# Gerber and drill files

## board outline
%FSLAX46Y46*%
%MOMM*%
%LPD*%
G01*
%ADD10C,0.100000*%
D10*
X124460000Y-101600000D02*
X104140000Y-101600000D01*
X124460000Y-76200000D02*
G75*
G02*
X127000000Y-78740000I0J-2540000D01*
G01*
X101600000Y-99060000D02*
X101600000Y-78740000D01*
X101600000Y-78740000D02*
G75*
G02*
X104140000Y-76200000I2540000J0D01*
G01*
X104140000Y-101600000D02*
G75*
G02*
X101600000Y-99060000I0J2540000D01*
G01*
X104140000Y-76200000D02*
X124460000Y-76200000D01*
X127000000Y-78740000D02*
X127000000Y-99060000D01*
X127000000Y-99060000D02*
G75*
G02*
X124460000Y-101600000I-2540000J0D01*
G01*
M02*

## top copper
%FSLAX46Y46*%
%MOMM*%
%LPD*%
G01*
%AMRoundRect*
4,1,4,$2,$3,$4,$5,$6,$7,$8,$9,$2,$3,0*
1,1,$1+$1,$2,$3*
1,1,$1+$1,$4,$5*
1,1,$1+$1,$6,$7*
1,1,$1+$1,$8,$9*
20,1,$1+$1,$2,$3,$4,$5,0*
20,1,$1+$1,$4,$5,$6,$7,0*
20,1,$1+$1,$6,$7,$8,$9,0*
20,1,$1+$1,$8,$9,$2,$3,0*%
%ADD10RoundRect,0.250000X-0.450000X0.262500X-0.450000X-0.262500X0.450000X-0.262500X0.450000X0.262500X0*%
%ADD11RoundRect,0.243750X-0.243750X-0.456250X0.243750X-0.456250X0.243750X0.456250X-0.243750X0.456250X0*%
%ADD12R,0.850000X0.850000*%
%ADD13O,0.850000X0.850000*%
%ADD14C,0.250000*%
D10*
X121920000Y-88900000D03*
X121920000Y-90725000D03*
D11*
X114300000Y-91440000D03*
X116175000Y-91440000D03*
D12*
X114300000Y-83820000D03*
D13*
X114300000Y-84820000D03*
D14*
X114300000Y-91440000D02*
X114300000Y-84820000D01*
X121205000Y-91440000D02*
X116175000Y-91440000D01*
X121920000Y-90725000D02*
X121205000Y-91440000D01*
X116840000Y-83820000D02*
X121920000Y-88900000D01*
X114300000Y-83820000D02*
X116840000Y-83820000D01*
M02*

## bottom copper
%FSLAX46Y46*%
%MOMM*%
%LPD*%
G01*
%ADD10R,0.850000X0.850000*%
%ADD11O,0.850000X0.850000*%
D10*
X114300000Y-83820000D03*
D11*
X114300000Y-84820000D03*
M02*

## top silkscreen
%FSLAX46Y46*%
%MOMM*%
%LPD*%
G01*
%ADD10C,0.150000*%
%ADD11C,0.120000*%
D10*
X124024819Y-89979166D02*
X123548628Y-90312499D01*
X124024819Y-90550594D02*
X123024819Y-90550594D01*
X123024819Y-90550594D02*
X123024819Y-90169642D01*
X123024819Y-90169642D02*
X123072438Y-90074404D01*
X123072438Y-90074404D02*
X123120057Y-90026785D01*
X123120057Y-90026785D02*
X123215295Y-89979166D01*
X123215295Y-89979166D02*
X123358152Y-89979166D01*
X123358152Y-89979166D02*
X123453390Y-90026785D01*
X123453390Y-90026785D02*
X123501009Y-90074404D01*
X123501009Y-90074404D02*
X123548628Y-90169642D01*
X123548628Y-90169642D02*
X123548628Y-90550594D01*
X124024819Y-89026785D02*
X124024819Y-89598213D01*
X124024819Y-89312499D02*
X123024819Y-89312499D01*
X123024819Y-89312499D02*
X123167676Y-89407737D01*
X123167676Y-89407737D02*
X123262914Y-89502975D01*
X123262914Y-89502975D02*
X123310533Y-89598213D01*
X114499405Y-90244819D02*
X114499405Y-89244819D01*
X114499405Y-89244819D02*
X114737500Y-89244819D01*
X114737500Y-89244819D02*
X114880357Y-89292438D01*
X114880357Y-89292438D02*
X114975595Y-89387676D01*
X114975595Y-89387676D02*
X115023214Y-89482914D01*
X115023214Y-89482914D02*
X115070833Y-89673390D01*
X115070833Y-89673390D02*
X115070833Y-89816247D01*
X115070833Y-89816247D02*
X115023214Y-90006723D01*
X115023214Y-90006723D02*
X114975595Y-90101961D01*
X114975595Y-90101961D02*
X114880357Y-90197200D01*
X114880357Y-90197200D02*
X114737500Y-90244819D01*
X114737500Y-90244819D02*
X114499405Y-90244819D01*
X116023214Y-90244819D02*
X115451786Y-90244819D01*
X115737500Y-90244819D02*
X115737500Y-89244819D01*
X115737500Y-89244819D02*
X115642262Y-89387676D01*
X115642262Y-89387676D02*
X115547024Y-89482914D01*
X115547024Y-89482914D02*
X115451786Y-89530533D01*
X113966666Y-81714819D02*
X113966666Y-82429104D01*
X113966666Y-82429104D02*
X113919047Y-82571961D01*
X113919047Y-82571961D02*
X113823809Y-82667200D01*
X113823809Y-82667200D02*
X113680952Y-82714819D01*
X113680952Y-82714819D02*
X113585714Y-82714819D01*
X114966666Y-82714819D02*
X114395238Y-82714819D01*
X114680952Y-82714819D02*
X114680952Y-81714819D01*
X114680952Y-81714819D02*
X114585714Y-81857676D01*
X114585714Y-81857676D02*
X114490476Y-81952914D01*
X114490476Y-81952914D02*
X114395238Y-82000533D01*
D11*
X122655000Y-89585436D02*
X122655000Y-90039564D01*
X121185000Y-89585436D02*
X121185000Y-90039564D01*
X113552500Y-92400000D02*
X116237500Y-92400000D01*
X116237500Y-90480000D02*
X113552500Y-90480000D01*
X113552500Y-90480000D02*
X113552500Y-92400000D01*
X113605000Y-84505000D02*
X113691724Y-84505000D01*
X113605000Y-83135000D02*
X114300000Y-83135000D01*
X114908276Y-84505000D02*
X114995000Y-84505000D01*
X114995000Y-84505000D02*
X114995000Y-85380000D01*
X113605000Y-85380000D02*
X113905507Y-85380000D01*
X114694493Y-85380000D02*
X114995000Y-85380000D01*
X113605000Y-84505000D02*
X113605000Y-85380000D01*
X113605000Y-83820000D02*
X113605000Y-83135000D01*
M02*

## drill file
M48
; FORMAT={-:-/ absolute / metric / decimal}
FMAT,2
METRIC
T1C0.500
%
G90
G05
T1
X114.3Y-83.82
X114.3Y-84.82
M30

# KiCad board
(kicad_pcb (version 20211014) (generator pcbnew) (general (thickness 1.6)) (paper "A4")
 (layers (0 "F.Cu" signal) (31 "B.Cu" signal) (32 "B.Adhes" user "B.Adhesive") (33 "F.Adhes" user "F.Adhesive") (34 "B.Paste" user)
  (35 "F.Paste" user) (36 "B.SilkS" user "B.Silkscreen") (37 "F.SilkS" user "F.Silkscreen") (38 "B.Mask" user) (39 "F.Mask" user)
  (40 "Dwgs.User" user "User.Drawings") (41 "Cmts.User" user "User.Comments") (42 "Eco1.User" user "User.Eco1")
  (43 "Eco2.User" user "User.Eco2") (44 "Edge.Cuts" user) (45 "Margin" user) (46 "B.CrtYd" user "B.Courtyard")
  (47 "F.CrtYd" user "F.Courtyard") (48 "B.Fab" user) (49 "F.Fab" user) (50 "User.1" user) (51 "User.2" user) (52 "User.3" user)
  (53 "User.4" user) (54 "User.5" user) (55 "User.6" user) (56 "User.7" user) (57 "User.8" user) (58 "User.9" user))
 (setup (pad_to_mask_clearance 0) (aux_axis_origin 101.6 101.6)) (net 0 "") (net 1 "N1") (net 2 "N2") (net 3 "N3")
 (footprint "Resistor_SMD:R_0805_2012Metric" (layer "F.Cu") (at 121.92 89.8125 -90)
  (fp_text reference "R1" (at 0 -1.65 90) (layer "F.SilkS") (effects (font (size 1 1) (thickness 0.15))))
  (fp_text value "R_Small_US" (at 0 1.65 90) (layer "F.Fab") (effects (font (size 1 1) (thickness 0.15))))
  (fp_line (start -0.227064 -0.735) (end 0.227064 -0.735) (layer "F.SilkS") (width 0.12))
  (fp_line (start -0.227064 0.735) (end 0.227064 0.735) (layer "F.SilkS") (width 0.12))
  (pad "1" smd roundrect (at -0.9125 0 270) (size 1.025 1.4) (layers "F.Cu" "F.Paste" "F.Mask") (roundrect_rratio 0.243902) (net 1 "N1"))
  (pad "2" smd roundrect (at 0.9125 0 270) (size 1.025 1.4) (layers "F.Cu" "F.Paste" "F.Mask") (roundrect_rratio 0.243902) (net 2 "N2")))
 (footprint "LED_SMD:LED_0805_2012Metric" (layer "F.Cu") (at 115.2375 91.44)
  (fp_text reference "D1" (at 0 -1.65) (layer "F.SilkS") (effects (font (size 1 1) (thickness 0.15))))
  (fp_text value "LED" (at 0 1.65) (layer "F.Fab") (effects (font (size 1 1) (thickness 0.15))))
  (fp_line (start -1.685 0.96) (end 1 0.96) (layer "F.SilkS") (width 0.12))
  (fp_line (start 1 -0.96) (end -1.685 -0.96) (layer "F.SilkS") (width 0.12))
  (fp_line (start -1.685 -0.96) (end -1.685 0.96) (layer "F.SilkS") (width 0.12))
  (pad "1" smd roundrect (at -0.9375 0) (size 0.975 1.4) (layers "F.Cu" "F.Paste" "F.Mask") (roundrect_rratio 0.25) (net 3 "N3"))
  (pad "2" smd roundrect (at 0.9375 0) (size 0.975 1.4) (layers "F.Cu" "F.Paste" "F.Mask") (roundrect_rratio 0.25) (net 2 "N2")))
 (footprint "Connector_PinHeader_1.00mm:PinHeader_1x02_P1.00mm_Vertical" (layer "F.Cu") (at 114.3 83.82)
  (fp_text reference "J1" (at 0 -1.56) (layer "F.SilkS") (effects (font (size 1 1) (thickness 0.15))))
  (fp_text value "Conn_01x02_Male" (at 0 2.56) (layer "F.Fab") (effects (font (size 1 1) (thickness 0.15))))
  (fp_line (start -0.695 0.685) (end -0.608276 0.685) (layer "F.SilkS") (width 0.12))
  (fp_line (start -0.695 -0.685) (end 0 -0.685) (layer "F.SilkS") (width 0.12))
  (fp_line (start 0.608276 0.685) (end 0.695 0.685) (layer "F.SilkS") (width 0.12))
  (fp_line (start 0.695 0.685) (end 0.695 1.56) (layer "F.SilkS") (width 0.12))
  (fp_line (start -0.695 1.56) (end -0.394493 1.56) (layer "F.SilkS") (width 0.12))
  (fp_line (start 0.394493 1.56) (end 0.695 1.56) (layer "F.SilkS") (width 0.12))
  (fp_line (start -0.695 0.685) (end -0.695 1.56) (layer "F.SilkS") (width 0.12))
  (fp_line (start -0.695 0) (end -0.695 -0.685) (layer "F.SilkS") (width 0.12))
  (pad "1" thru_hole rect (at 0 0) (size 0.85 0.85) (drill 0.5) (layers *.Cu *.Mask) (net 1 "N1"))
  (pad "2" thru_hole oval (at 0 1) (size 0.85 0.85) (drill 0.5) (layers *.Cu *.Mask) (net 3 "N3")))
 (gr_line (start 124.46 101.6) (end 104.14 101.6) (layer "Edge.Cuts") (width 0.1))
 (gr_arc (start 124.46 76.2) (mid 126.256051 76.943949) (end 127 78.74) (layer "Edge.Cuts") (width 0.1))
 (gr_line (start 101.6 99.06) (end 101.6 78.74) (layer "Edge.Cuts") (width 0.1))
 (gr_arc (start 101.6 78.74) (mid 102.343949 76.943949) (end 104.14 76.2) (layer "Edge.Cuts") (width 0.1))
 (gr_arc (start 104.14 101.6) (mid 102.343949 100.856051) (end 101.6 99.06) (layer "Edge.Cuts") (width 0.1))
 (gr_line (start 104.14 76.2) (end 124.46 76.2) (layer "Edge.Cuts") (width 0.1))
 (gr_line (start 127 78.74) (end 127 99.06) (layer "Edge.Cuts") (width 0.1))
 (gr_arc (start 127 99.06) (mid 126.256051 100.856051) (end 124.46 101.6) (layer "Edge.Cuts") (width 0.1))
 (segment (start 114.3 91.44) (end 114.3 84.82) (width 0.25) (layer "F.Cu") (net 3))
 (segment (start 121.205 91.44) (end 116.175 91.44) (width 0.25) (layer "F.Cu") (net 2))
 (segment (start 121.92 90.725) (end 121.205 91.44) (width 0.25) (layer "F.Cu") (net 2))
 (segment (start 116.84 83.82) (end 121.92 88.9) (width 0.25) (layer "F.Cu") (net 1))
 (segment (start 114.3 83.82) (end 116.84 83.82) (width 0.25) (layer "F.Cu") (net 1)))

